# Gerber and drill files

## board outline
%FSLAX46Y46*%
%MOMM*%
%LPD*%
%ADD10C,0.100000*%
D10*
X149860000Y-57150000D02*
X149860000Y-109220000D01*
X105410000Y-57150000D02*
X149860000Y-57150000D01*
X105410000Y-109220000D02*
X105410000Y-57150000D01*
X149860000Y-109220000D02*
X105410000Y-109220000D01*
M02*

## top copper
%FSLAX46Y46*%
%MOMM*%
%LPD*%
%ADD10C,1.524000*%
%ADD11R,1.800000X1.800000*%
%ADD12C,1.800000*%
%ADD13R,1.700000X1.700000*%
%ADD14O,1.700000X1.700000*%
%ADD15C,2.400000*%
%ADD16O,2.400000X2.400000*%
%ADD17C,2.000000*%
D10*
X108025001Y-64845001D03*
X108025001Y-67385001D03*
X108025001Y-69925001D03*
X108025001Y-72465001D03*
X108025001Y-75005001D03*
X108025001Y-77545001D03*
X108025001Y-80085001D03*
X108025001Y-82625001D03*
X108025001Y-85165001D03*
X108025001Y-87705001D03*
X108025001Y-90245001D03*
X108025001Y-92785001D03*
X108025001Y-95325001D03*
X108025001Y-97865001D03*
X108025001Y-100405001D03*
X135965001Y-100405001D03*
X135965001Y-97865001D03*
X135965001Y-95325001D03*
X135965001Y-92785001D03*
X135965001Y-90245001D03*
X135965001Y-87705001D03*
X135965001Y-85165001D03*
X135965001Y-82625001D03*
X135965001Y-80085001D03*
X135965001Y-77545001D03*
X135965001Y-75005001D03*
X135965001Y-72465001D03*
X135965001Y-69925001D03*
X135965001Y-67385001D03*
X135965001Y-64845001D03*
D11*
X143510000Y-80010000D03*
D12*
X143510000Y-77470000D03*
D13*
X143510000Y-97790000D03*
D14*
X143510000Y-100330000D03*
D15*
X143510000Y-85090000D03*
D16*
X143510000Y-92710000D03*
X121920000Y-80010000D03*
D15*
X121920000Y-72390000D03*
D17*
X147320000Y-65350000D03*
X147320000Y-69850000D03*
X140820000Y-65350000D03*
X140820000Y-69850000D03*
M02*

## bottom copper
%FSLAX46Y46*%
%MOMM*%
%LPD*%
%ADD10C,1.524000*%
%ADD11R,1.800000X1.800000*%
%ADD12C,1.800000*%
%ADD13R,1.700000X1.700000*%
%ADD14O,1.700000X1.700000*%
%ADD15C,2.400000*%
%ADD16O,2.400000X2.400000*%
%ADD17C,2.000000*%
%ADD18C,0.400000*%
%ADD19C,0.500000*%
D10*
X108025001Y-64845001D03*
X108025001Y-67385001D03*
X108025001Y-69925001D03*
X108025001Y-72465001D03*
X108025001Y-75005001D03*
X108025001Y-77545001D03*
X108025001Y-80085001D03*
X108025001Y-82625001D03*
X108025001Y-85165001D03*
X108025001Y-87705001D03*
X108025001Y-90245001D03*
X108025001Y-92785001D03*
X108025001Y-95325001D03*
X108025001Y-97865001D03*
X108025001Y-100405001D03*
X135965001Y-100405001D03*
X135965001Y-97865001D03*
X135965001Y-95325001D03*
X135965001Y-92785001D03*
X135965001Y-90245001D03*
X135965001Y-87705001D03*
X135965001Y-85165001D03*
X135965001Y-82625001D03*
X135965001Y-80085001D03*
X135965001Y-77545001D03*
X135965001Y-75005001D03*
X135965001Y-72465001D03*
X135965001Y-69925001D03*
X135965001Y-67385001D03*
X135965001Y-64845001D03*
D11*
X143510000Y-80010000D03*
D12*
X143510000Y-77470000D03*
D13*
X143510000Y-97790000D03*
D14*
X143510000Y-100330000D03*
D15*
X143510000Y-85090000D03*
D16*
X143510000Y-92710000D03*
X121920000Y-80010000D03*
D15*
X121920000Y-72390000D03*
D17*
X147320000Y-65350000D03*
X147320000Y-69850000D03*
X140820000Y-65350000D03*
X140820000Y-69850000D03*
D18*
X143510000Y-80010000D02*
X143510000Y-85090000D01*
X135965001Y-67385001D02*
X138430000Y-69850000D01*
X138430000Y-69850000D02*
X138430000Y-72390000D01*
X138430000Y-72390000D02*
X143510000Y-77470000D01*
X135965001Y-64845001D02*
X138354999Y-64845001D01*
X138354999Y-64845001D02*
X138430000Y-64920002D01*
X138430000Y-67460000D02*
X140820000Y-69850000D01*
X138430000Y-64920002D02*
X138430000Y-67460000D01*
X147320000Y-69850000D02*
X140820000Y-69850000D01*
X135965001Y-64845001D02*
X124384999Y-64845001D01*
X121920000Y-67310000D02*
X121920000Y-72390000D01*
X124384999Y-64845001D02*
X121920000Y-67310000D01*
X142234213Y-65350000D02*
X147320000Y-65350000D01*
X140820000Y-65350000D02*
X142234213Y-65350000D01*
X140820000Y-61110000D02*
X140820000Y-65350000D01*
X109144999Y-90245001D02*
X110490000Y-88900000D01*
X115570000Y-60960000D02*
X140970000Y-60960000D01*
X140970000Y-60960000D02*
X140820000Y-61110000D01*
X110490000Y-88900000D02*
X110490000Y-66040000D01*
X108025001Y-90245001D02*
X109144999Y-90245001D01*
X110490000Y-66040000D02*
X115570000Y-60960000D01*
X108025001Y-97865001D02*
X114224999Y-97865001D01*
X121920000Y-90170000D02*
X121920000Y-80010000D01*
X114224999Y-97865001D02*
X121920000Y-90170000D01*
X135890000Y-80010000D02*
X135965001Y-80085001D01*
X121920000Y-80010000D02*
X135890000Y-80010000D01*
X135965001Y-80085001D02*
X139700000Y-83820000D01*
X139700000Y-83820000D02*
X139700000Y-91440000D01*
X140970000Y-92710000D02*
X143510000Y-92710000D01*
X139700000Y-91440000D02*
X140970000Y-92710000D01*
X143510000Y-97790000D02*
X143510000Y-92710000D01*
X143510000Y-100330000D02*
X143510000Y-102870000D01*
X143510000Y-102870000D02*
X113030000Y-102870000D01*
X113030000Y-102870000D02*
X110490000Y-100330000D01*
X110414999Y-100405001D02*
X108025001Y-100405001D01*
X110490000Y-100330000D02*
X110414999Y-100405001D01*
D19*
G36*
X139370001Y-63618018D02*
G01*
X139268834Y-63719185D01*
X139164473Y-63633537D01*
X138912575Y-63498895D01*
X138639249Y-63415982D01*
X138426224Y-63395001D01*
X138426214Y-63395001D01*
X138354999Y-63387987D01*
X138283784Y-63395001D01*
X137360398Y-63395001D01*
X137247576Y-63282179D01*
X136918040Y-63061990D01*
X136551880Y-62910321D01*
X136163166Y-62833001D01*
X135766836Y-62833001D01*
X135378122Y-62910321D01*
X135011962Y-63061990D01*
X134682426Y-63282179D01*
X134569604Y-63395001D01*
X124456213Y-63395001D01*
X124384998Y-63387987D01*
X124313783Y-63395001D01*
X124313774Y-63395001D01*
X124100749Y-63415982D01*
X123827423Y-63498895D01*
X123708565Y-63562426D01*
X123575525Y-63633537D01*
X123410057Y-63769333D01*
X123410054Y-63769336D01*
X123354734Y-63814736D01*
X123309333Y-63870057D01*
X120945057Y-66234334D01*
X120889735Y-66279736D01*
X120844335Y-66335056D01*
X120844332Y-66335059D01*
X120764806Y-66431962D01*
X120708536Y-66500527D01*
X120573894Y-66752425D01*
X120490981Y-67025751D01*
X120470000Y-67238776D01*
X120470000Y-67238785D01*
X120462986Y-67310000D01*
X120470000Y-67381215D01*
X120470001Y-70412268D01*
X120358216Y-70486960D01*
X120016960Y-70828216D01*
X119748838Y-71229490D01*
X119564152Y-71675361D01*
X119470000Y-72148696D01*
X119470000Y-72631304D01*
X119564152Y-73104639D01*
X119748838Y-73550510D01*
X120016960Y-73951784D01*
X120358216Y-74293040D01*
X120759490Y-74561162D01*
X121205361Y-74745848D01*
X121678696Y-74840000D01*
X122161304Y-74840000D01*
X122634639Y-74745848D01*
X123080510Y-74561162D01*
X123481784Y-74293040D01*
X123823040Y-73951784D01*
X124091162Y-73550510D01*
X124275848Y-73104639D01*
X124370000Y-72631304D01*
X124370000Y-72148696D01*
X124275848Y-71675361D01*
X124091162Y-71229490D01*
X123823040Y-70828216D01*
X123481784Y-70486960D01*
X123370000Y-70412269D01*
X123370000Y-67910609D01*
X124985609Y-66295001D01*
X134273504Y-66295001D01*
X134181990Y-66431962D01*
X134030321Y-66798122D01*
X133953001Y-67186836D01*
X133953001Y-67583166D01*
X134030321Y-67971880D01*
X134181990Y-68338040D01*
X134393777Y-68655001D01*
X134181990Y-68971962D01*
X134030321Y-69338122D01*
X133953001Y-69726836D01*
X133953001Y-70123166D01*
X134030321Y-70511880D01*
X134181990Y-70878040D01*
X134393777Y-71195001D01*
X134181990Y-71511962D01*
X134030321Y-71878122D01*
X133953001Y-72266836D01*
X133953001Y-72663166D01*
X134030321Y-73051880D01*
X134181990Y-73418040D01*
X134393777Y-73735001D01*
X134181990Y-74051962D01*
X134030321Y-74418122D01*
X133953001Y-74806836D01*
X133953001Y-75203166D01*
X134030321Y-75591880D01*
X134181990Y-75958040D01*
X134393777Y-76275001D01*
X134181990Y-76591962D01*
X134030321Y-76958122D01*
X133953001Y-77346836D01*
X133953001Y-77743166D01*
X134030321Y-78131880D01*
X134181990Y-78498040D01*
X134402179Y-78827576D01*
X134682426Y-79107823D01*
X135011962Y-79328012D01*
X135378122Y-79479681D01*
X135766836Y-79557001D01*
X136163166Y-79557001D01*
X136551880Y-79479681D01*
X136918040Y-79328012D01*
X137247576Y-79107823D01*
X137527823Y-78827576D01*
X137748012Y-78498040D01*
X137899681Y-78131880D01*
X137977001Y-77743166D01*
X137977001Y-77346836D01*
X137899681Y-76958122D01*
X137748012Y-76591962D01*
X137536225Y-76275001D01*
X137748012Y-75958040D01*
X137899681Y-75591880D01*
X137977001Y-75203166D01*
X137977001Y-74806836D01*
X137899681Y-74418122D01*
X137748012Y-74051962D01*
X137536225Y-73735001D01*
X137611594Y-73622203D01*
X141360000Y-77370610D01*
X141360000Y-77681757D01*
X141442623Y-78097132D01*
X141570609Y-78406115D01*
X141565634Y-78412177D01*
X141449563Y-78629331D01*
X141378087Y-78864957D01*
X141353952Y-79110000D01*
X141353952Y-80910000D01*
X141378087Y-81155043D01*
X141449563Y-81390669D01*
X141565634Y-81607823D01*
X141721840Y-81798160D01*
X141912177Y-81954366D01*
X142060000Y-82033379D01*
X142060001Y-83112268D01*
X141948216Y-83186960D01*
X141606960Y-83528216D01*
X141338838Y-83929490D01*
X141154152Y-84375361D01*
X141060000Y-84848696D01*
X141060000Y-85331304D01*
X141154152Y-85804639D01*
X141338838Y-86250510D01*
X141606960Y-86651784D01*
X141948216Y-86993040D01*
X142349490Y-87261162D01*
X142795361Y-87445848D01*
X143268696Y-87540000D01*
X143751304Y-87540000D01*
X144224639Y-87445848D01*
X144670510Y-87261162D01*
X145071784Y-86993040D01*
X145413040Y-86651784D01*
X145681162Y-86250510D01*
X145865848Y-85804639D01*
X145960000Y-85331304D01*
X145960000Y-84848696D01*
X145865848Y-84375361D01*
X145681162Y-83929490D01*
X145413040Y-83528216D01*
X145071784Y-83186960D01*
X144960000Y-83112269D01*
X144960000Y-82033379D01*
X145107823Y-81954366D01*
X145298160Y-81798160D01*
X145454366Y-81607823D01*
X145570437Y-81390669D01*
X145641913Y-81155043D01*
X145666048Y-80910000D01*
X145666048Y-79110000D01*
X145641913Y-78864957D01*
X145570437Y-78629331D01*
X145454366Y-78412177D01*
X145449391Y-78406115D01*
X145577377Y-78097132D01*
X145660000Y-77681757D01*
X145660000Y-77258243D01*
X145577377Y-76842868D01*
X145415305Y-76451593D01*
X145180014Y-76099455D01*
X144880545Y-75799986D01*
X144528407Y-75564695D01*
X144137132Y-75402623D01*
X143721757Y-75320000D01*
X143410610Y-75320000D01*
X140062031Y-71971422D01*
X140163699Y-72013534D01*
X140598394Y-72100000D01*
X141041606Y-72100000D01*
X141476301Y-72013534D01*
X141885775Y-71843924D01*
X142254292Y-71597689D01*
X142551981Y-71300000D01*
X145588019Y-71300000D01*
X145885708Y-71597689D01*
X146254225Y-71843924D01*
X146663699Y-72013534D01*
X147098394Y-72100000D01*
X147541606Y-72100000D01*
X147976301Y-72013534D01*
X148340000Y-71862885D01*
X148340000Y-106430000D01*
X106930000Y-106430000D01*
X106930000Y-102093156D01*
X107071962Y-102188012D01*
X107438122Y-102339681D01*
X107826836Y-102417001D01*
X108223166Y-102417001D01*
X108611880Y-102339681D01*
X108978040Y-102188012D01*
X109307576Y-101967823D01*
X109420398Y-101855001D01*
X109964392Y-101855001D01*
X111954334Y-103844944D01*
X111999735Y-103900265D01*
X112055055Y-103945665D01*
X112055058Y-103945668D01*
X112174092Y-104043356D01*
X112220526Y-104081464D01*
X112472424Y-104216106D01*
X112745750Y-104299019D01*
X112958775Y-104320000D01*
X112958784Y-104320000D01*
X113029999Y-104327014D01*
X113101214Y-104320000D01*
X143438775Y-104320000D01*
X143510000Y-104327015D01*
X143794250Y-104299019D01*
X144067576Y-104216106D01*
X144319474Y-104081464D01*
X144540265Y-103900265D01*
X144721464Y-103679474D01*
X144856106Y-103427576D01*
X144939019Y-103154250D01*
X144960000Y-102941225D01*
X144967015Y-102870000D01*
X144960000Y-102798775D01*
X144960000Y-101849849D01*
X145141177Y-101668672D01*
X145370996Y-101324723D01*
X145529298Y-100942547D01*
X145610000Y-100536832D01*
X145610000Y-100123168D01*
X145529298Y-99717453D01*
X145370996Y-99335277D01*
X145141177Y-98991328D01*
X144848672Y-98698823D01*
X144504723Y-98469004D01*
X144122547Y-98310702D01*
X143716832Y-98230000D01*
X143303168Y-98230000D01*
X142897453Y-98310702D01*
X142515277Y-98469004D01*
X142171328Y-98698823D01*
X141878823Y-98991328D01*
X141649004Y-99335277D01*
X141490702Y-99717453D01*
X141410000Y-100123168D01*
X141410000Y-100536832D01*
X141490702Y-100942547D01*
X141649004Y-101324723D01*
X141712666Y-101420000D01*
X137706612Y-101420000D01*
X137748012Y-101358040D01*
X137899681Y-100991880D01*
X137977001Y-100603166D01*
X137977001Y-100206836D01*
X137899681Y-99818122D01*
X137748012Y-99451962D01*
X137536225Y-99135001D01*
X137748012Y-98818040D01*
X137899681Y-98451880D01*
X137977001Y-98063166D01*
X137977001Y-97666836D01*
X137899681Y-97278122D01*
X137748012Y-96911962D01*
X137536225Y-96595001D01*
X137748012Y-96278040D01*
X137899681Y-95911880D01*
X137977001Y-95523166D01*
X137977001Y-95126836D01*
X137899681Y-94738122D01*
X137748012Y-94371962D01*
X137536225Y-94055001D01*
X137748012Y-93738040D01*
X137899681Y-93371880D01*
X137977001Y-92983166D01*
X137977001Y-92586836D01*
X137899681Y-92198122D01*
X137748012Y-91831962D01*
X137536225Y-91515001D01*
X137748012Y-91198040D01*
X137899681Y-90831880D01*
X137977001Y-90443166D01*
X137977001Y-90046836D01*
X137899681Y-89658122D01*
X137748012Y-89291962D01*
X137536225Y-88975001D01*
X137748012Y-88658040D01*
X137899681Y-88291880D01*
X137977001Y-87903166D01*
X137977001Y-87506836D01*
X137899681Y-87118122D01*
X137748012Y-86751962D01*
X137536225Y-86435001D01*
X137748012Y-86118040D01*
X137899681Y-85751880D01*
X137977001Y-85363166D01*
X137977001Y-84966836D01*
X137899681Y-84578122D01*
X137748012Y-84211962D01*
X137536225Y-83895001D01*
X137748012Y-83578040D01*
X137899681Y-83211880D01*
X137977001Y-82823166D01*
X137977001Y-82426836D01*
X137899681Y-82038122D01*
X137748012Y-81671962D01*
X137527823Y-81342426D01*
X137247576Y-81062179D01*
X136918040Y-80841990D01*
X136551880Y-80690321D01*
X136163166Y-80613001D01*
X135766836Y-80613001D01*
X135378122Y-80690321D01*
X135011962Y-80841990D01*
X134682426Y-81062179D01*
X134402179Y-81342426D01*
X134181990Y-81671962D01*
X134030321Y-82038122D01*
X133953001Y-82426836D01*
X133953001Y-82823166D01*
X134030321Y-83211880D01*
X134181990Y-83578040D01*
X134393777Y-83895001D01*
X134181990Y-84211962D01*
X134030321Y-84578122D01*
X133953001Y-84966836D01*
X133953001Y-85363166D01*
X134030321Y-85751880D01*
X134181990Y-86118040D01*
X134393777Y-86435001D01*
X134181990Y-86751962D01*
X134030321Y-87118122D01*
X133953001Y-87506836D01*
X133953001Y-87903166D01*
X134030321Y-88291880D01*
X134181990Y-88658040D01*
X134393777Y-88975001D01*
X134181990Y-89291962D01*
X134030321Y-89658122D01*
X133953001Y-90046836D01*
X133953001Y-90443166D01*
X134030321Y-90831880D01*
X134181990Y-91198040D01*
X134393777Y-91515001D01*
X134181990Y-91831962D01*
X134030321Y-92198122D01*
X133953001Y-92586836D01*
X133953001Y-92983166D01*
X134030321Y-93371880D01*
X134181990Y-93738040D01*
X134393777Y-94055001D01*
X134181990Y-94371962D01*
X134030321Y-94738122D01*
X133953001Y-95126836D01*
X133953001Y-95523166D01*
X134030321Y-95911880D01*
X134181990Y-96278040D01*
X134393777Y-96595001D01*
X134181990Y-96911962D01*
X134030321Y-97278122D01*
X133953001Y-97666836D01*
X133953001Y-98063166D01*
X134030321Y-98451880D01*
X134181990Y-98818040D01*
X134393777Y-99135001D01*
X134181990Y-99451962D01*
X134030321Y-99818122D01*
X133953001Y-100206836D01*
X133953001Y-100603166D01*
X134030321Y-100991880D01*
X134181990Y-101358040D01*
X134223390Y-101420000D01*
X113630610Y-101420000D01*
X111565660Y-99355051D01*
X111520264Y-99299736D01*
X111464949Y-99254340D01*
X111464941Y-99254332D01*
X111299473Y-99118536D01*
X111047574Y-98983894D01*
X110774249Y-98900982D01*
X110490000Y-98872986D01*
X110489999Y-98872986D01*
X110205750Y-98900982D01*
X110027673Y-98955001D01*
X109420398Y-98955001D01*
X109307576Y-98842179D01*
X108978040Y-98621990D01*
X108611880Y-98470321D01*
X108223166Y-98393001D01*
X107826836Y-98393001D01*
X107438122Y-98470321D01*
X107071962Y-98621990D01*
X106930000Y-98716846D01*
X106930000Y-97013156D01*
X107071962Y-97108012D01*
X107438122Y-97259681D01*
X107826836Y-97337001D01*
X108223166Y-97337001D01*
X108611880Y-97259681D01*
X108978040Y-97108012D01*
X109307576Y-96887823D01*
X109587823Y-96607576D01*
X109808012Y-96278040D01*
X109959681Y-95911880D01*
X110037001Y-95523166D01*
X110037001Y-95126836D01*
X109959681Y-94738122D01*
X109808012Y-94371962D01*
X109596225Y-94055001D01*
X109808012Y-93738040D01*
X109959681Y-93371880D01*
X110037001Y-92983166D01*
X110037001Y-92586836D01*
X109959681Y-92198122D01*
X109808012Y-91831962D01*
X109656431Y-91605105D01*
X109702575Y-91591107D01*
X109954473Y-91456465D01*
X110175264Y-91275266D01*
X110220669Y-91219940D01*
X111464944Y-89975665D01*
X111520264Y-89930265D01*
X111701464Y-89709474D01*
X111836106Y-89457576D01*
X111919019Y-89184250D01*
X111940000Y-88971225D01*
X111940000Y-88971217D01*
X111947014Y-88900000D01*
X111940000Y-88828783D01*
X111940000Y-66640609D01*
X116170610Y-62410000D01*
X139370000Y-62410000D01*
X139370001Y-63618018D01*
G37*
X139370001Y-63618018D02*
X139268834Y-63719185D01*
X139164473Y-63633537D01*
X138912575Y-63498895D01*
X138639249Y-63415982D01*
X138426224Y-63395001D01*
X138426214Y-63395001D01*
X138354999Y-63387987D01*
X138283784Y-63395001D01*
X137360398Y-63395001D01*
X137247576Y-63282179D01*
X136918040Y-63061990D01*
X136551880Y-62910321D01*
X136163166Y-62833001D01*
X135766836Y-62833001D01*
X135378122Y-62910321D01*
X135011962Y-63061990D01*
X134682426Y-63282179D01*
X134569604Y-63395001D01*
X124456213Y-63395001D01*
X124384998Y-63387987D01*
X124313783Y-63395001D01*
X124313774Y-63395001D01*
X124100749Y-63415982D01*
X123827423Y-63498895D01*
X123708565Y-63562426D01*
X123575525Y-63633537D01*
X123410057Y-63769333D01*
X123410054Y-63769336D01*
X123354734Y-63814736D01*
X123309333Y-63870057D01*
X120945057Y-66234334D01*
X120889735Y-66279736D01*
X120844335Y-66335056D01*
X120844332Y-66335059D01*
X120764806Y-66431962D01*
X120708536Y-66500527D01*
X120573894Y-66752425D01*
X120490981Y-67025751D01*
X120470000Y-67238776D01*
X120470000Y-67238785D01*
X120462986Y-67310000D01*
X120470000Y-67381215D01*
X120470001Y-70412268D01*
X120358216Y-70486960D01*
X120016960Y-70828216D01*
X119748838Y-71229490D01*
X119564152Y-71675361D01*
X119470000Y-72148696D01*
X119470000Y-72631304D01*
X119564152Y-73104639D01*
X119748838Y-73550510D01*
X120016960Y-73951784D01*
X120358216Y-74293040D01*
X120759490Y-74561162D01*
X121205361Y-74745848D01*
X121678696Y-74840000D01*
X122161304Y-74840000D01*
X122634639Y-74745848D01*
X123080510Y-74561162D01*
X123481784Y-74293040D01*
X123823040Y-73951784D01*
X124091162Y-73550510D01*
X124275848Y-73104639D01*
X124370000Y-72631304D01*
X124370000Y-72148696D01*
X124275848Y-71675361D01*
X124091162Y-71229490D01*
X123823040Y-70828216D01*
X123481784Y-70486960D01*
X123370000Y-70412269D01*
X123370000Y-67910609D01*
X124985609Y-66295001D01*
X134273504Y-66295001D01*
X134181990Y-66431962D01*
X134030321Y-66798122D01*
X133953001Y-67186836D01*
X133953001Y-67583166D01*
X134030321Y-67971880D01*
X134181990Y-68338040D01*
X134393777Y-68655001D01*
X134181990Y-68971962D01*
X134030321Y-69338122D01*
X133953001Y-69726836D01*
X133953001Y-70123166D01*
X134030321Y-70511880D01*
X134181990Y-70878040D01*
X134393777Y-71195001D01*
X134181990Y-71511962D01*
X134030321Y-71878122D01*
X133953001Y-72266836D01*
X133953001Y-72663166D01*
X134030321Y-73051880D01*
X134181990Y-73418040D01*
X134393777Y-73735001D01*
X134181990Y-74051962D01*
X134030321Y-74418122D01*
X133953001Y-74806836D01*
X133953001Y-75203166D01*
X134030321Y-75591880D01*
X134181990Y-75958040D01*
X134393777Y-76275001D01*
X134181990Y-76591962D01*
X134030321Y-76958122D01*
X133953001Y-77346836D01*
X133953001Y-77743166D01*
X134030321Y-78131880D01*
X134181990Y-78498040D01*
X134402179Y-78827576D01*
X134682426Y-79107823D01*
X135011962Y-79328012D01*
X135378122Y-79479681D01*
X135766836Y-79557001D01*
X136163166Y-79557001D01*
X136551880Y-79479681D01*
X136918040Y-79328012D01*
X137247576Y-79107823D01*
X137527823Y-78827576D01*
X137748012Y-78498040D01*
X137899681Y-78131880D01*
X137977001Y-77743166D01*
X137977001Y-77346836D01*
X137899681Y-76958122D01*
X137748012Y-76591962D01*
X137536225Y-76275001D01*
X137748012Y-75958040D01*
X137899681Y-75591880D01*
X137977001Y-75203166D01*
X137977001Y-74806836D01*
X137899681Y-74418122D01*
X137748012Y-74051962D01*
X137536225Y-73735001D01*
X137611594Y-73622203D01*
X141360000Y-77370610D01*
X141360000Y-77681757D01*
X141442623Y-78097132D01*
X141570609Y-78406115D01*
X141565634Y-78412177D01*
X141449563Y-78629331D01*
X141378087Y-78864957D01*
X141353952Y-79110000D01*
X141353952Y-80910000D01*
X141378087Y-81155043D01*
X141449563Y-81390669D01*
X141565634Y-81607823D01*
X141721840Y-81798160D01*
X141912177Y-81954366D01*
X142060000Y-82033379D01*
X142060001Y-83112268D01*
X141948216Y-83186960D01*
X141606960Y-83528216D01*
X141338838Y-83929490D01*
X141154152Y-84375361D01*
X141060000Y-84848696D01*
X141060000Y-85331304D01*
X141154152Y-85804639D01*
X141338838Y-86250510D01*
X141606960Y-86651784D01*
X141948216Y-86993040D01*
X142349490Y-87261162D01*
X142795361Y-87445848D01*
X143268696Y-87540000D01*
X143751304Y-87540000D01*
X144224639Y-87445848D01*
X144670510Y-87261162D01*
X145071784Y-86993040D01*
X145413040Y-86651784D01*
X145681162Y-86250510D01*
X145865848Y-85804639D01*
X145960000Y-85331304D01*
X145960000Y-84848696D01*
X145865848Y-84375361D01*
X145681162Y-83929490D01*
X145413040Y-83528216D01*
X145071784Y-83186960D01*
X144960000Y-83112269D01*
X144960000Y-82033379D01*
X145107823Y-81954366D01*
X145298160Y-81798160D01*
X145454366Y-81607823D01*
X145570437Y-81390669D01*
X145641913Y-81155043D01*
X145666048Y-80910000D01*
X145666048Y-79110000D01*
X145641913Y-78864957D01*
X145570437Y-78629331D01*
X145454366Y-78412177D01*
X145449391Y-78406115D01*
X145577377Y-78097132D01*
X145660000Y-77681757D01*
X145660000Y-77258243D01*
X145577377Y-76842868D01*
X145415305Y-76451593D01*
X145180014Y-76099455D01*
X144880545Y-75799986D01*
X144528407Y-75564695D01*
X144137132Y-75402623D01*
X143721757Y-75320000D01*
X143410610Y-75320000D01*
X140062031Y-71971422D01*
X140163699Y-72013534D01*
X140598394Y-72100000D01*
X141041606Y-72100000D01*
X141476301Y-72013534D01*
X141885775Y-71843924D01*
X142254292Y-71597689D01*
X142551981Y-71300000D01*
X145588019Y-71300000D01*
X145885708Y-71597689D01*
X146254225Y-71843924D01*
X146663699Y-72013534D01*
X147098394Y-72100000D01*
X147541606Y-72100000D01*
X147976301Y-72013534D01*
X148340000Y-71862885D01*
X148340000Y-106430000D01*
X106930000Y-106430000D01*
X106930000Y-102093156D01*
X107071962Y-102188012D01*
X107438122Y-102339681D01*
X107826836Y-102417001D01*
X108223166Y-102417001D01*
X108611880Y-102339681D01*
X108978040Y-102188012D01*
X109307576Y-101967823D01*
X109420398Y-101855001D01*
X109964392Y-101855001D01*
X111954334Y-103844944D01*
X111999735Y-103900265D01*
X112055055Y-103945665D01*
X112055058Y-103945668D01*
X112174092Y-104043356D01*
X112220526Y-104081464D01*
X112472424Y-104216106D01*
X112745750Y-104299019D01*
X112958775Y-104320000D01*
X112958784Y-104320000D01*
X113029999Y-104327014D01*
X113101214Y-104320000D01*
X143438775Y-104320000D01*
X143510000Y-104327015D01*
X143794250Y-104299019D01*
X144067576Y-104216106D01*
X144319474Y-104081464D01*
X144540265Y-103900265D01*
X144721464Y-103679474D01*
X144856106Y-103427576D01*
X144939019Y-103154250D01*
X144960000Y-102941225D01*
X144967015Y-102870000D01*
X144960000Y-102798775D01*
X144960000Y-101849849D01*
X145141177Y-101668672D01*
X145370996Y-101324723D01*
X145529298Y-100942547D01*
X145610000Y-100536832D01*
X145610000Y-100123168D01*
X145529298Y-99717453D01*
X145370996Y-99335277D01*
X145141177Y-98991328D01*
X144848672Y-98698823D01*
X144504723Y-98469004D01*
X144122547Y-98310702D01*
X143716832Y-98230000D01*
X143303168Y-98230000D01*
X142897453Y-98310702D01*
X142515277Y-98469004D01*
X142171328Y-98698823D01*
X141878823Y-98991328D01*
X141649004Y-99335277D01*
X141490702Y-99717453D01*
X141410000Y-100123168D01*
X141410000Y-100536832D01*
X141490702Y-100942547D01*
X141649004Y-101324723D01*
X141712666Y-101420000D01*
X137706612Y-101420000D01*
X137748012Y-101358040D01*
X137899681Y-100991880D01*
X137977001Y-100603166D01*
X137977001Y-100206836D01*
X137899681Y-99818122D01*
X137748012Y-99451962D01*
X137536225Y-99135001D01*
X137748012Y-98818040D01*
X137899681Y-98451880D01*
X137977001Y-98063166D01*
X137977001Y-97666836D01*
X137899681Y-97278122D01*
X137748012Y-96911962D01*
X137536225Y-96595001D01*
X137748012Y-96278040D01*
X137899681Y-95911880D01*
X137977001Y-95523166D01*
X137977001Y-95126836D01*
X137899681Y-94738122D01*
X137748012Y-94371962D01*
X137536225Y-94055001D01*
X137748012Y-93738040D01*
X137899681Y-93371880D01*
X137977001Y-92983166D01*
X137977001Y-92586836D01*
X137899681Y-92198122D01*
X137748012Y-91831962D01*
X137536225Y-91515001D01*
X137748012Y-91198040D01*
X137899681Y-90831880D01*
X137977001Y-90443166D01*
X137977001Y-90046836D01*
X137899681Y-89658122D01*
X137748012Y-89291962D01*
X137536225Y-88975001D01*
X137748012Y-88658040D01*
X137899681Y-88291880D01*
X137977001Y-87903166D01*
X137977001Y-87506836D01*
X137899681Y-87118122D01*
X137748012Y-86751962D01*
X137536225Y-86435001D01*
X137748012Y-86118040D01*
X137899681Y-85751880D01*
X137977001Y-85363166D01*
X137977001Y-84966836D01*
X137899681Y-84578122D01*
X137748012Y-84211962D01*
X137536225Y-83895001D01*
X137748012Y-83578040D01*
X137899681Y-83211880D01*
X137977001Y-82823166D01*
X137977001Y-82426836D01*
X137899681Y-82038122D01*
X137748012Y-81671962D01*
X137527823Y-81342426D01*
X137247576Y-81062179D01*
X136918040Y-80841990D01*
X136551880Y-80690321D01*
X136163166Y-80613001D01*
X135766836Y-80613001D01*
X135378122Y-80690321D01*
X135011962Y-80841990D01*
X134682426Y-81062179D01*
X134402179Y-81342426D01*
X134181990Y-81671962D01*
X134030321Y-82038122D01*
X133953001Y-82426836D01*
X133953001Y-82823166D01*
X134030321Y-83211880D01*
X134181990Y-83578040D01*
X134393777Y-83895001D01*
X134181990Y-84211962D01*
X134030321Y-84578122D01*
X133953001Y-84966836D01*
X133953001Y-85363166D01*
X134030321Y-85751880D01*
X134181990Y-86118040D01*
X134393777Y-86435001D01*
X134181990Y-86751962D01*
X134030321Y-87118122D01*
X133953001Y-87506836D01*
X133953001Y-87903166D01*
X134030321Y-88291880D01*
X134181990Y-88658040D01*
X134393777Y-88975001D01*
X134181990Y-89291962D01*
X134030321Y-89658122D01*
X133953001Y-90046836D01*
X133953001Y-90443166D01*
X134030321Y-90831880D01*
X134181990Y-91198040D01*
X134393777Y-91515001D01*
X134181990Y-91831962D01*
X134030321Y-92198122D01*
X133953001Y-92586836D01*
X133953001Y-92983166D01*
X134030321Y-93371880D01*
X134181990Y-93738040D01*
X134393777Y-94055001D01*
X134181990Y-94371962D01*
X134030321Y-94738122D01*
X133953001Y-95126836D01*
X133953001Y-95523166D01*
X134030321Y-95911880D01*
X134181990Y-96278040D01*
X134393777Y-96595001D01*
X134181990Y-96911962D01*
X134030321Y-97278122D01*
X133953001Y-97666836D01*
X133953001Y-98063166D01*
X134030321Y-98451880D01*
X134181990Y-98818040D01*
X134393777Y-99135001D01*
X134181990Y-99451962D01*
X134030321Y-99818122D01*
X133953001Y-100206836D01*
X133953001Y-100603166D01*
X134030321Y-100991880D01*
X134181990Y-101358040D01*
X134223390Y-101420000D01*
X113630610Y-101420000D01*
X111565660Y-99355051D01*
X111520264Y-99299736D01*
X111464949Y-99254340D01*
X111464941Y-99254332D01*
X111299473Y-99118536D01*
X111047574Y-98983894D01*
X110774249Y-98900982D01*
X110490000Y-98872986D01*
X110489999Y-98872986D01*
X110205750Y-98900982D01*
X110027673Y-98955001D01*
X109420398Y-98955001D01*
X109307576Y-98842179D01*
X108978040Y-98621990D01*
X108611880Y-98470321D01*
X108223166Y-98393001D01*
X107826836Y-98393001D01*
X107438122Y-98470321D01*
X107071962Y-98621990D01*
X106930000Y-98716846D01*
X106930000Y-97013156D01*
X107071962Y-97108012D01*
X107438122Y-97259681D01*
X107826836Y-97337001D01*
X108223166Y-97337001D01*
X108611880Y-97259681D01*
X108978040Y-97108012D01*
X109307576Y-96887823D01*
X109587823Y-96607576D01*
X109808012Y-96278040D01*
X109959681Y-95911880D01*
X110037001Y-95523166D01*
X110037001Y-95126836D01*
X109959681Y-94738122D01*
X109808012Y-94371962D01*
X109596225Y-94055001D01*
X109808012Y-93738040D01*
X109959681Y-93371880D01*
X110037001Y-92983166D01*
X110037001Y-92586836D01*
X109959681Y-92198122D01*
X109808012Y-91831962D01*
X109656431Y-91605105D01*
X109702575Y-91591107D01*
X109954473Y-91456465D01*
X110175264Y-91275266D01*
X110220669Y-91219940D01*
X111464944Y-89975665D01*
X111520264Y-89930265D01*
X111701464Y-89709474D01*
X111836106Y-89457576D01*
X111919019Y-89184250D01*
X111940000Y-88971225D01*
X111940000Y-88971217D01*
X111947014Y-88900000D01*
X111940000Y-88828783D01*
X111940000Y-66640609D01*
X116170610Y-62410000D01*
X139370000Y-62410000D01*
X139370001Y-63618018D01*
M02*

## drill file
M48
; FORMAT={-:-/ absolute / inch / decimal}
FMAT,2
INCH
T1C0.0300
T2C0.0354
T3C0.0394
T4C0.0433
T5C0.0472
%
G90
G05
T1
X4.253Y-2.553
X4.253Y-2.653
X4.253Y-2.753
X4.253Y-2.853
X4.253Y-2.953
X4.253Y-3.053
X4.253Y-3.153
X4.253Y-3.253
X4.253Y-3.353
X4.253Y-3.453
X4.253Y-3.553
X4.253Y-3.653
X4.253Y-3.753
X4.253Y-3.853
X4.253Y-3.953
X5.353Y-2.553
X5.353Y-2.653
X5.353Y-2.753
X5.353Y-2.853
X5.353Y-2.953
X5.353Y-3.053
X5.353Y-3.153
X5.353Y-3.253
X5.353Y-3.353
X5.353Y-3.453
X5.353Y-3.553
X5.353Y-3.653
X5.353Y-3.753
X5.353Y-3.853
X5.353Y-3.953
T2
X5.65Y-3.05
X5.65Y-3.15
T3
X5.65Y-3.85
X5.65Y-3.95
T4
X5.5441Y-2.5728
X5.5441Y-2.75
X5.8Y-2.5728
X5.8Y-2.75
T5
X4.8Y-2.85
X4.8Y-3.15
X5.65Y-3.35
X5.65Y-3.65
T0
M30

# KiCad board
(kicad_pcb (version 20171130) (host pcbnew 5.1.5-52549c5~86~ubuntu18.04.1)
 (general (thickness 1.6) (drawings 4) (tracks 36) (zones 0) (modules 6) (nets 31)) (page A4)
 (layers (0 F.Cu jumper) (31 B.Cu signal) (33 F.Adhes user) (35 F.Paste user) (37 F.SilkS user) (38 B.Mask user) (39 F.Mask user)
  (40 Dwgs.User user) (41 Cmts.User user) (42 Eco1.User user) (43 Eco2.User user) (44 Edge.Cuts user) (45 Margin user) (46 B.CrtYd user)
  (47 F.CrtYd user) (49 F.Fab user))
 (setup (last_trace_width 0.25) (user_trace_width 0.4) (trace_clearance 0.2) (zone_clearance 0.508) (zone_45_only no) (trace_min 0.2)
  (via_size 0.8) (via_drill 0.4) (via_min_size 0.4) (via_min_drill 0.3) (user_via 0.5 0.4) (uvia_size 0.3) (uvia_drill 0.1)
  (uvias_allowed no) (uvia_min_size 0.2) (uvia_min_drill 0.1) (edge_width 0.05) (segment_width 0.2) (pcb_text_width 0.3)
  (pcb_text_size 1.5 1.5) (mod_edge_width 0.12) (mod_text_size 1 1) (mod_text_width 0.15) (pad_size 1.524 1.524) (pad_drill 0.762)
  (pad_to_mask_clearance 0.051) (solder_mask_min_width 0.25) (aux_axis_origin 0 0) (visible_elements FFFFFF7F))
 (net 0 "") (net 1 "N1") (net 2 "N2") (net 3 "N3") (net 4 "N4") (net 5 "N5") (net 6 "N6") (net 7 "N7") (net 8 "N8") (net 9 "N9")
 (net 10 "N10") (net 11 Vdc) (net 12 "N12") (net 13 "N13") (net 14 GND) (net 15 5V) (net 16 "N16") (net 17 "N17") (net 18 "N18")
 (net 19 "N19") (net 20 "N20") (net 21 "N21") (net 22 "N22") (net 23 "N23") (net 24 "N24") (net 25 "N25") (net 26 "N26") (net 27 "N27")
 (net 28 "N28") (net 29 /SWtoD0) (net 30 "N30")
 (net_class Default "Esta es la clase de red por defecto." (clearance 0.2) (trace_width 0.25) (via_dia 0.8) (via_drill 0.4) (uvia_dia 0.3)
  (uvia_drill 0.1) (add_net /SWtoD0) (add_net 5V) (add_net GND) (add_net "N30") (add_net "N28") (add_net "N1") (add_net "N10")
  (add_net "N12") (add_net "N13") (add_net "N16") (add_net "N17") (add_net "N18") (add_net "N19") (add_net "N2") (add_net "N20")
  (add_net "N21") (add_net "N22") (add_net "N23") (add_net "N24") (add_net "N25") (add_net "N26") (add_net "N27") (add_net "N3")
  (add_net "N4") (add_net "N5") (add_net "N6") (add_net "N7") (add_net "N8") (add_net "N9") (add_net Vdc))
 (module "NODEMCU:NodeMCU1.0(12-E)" (layer F.Cu) (at 121.995001 82.625001)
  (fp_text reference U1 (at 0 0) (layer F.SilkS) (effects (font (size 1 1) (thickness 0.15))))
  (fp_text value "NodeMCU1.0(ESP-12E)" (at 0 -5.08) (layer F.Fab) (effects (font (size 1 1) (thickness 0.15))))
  (pad 1 thru_hole circle (at -13.97 -17.78) (size 1.524 1.524) (drill 0.762) (layers *.Cu *.Mask F.SilkS) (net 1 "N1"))
  (pad 2 thru_hole circle (at -13.97 -15.24) (size 1.524 1.524) (drill 0.762) (layers *.Cu *.Mask F.SilkS) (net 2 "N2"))
  (pad 3 thru_hole circle (at -13.97 -12.7) (size 1.524 1.524) (drill 0.762) (layers *.Cu *.Mask F.SilkS) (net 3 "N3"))
  (pad 4 thru_hole circle (at -13.97 -10.16) (size 1.524 1.524) (drill 0.762) (layers *.Cu *.Mask F.SilkS) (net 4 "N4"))
  (pad 5 thru_hole circle (at -13.97 -7.62) (size 1.524 1.524) (drill 0.762) (layers *.Cu *.Mask F.SilkS) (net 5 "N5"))
  (pad 6 thru_hole circle (at -13.97 -5.08) (size 1.524 1.524) (drill 0.762) (layers *.Cu *.Mask F.SilkS) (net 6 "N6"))
  (pad 7 thru_hole circle (at -13.97 -2.54) (size 1.524 1.524) (drill 0.762) (layers *.Cu *.Mask F.SilkS) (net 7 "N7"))
  (pad 8 thru_hole circle (at -13.97 0) (size 1.524 1.524) (drill 0.762) (layers *.Cu *.Mask F.SilkS) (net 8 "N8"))
  (pad 9 thru_hole circle (at -13.97 2.54) (size 1.524 1.524) (drill 0.762) (layers *.Cu *.Mask F.SilkS) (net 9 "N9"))
  (pad 10 thru_hole circle (at -13.97 5.08) (size 1.524 1.524) (drill 0.762) (layers *.Cu *.Mask F.SilkS) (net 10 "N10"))
  (pad 11 thru_hole circle (at -13.97 7.62) (size 1.524 1.524) (drill 0.762) (layers *.Cu *.Mask F.SilkS) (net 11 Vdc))
  (pad 12 thru_hole circle (at -13.97 10.16) (size 1.524 1.524) (drill 0.762) (layers *.Cu *.Mask F.SilkS) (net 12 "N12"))
  (pad 13 thru_hole circle (at -13.97 12.7) (size 1.524 1.524) (drill 0.762) (layers *.Cu *.Mask F.SilkS) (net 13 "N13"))
  (pad 14 thru_hole circle (at -13.97 15.24) (size 1.524 1.524) (drill 0.762) (layers *.Cu *.Mask F.SilkS) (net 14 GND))
  (pad 15 thru_hole circle (at -13.97 17.78) (size 1.524 1.524) (drill 0.762) (layers *.Cu *.Mask F.SilkS) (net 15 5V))
  (pad 16 thru_hole circle (at 13.97 17.78) (size 1.524 1.524) (drill 0.762) (layers *.Cu *.Mask F.SilkS) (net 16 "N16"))
  (pad 17 thru_hole circle (at 13.97 15.24) (size 1.524 1.524) (drill 0.762) (layers *.Cu *.Mask F.SilkS) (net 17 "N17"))
  (pad 18 thru_hole circle (at 13.97 12.7) (size 1.524 1.524) (drill 0.762) (layers *.Cu *.Mask F.SilkS) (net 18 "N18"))
  (pad 19 thru_hole circle (at 13.97 10.16) (size 1.524 1.524) (drill 0.762) (layers *.Cu *.Mask F.SilkS) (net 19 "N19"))
  (pad 20 thru_hole circle (at 13.97 7.62) (size 1.524 1.524) (drill 0.762) (layers *.Cu *.Mask F.SilkS) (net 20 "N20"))
  (pad 21 thru_hole circle (at 13.97 5.08) (size 1.524 1.524) (drill 0.762) (layers *.Cu *.Mask F.SilkS) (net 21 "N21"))
  (pad 22 thru_hole circle (at 13.97 2.54) (size 1.524 1.524) (drill 0.762) (layers *.Cu *.Mask F.SilkS) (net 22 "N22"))
  (pad 23 thru_hole circle (at 13.97 0) (size 1.524 1.524) (drill 0.762) (layers *.Cu *.Mask F.SilkS) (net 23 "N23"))
  (pad 24 thru_hole circle (at 13.97 -2.54) (size 1.524 1.524) (drill 0.762) (layers *.Cu *.Mask F.SilkS) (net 14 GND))
  (pad 25 thru_hole circle (at 13.97 -5.08) (size 1.524 1.524) (drill 0.762) (layers *.Cu *.Mask F.SilkS) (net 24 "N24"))
  (pad 26 thru_hole circle (at 13.97 -7.62) (size 1.524 1.524) (drill 0.762) (layers *.Cu *.Mask F.SilkS) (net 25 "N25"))
  (pad 27 thru_hole circle (at 13.97 -10.16) (size 1.524 1.524) (drill 0.762) (layers *.Cu *.Mask F.SilkS) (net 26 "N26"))
  (pad 28 thru_hole circle (at 13.97 -12.7) (size 1.524 1.524) (drill 0.762) (layers *.Cu *.Mask F.SilkS) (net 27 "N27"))
  (pad 29 thru_hole circle (at 13.97 -15.24) (size 1.524 1.524) (drill 0.762) (layers *.Cu *.Mask F.SilkS) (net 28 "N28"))
  (pad 30 thru_hole circle (at 13.97 -17.78) (size 1.524 1.524) (drill 0.762) (layers *.Cu *.Mask F.SilkS) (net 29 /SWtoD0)))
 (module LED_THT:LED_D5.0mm (layer F.Cu) (at 143.51 80.01 90)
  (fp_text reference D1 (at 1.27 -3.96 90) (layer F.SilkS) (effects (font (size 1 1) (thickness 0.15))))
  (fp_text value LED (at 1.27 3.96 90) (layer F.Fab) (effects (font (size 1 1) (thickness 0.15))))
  (pad 1 thru_hole rect (at 0 0 90) (size 1.8 1.8) (drill 0.9) (layers *.Cu *.Mask) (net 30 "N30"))
  (pad 2 thru_hole circle (at 2.54 0 90) (size 1.8 1.8) (drill 0.9) (layers *.Cu *.Mask) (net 28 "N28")))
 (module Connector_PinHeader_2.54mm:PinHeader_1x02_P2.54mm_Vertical (layer F.Cu) (at 143.51 97.79)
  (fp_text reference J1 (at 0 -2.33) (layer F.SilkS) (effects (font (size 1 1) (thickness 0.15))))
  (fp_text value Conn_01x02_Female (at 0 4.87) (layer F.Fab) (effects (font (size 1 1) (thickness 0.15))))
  (pad 1 thru_hole rect (at 0 0) (size 1.7 1.7) (drill 1) (layers *.Cu *.Mask) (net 14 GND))
  (pad 2 thru_hole oval (at 0 2.54) (size 1.7 1.7) (drill 1) (layers *.Cu *.Mask) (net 15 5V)))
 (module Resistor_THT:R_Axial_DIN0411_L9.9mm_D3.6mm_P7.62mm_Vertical (layer F.Cu) (at 143.51 85.09 270)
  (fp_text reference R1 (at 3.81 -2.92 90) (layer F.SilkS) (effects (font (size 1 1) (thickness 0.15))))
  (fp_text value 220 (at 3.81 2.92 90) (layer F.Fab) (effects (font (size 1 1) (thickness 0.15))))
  (pad 1 thru_hole circle (at 0 0 270) (size 2.4 2.4) (drill 1.2) (layers *.Cu *.Mask) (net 30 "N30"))
  (pad 2 thru_hole oval (at 7.62 0 270) (size 2.4 2.4) (drill 1.2) (layers *.Cu *.Mask) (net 14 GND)))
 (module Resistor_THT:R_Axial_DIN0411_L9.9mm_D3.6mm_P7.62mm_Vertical (layer F.Cu) (at 121.92 72.39 270)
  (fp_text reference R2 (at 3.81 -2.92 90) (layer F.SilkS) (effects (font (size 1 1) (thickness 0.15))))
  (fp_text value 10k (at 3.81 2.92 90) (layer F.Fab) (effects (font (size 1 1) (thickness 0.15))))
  (pad 2 thru_hole oval (at 7.62 0 270) (size 2.4 2.4) (drill 1.2) (layers *.Cu *.Mask) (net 14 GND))
  (pad 1 thru_hole circle (at 0 0 270) (size 2.4 2.4) (drill 1.2) (layers *.Cu *.Mask) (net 29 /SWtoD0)))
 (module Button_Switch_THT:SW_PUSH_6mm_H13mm (layer F.Cu) (at 147.32 69.85 180)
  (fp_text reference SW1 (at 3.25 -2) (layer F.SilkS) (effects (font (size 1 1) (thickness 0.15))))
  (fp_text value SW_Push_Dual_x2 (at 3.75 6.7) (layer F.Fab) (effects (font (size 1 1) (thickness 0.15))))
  (pad 2 thru_hole circle (at 0 4.5 270) (size 2 2) (drill 1.1) (layers *.Cu *.Mask) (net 11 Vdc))
  (pad 1 thru_hole circle (at 0 0 270) (size 2 2) (drill 1.1) (layers *.Cu *.Mask) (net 29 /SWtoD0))
  (pad 2 thru_hole circle (at 6.5 4.5 270) (size 2 2) (drill 1.1) (layers *.Cu *.Mask) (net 11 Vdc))
  (pad 1 thru_hole circle (at 6.5 0 270) (size 2 2) (drill 1.1) (layers *.Cu *.Mask) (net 29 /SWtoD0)))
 (gr_line (start 149.86 57.15) (end 149.86 109.22) (layer Edge.Cuts) (width 0.1))
 (gr_line (start 105.41 57.15) (end 149.86 57.15) (layer Edge.Cuts) (width 0.1))
 (gr_line (start 105.41 109.22) (end 105.41 57.15) (layer Edge.Cuts) (width 0.1))
 (gr_line (start 149.86 109.22) (end 105.41 109.22) (layer Edge.Cuts) (width 0.1))
 (segment (start 143.51 80.01) (end 143.51 85.09) (width 0.4) (layer B.Cu) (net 30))
 (segment (start 135.965001 67.385001) (end 138.43 69.85) (width 0.4) (layer B.Cu) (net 28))
 (segment (start 138.43 69.85) (end 138.43 72.39) (width 0.4) (layer B.Cu) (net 28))
 (segment (start 138.43 72.39) (end 143.51 77.47) (width 0.4) (layer B.Cu) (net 28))
 (segment (start 135.965001 64.845001) (end 138.354999 64.845001) (width 0.4) (layer B.Cu) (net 29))
 (segment (start 138.354999 64.845001) (end 138.43 64.920002) (width 0.4) (layer B.Cu) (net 29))
 (segment (start 138.43 67.46) (end 140.82 69.85) (width 0.4) (layer B.Cu) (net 29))
 (segment (start 138.43 64.920002) (end 138.43 67.46) (width 0.4) (layer B.Cu) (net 29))
 (segment (start 147.32 69.85) (end 140.82 69.85) (width 0.4) (layer B.Cu) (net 29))
 (segment (start 135.965001 64.845001) (end 124.384999 64.845001) (width 0.4) (layer B.Cu) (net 29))
 (segment (start 121.92 67.31) (end 121.92 72.39) (width 0.4) (layer B.Cu) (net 29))
 (segment (start 124.384999 64.845001) (end 121.92 67.31) (width 0.4) (layer B.Cu) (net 29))
 (segment (start 142.234213 65.35) (end 147.32 65.35) (width 0.4) (layer B.Cu) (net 11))
 (segment (start 140.82 65.35) (end 142.234213 65.35) (width 0.4) (layer B.Cu) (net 11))
 (segment (start 140.82 61.11) (end 140.82 65.35) (width 0.4) (layer B.Cu) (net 11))
 (segment (start 109.144999 90.245001) (end 110.49 88.9) (width 0.4) (layer B.Cu) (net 11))
 (segment (start 115.57 60.96) (end 140.97 60.96) (width 0.4) (layer B.Cu) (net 11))
 (segment (start 140.97 60.96) (end 140.82 61.11) (width 0.4) (layer B.Cu) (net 11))
 (segment (start 110.49 88.9) (end 110.49 66.04) (width 0.4) (layer B.Cu) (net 11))
 (segment (start 108.025001 90.245001) (end 109.144999 90.245001) (width 0.4) (layer B.Cu) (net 11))
 (segment (start 110.49 66.04) (end 115.57 60.96) (width 0.4) (layer B.Cu) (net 11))
 (segment (start 108.025001 97.865001) (end 114.224999 97.865001) (width 0.4) (layer B.Cu) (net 14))
 (segment (start 121.92 90.17) (end 121.92 80.01) (width 0.4) (layer B.Cu) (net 14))
 (segment (start 114.224999 97.865001) (end 121.92 90.17) (width 0.4) (layer B.Cu) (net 14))
 (segment (start 135.89 80.01) (end 135.965001 80.085001) (width 0.4) (layer B.Cu) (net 14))
 (segment (start 121.92 80.01) (end 135.89 80.01) (width 0.4) (layer B.Cu) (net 14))
 (segment (start 135.965001 80.085001) (end 139.7 83.82) (width 0.4) (layer B.Cu) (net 14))
 (segment (start 139.7 83.82) (end 139.7 91.44) (width 0.4) (layer B.Cu) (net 14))
 (segment (start 140.97 92.71) (end 143.51 92.71) (width 0.4) (layer B.Cu) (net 14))
 (segment (start 139.7 91.44) (end 140.97 92.71) (width 0.4) (layer B.Cu) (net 14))
 (segment (start 143.51 97.79) (end 143.51 92.71) (width 0.4) (layer B.Cu) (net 14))
 (segment (start 143.51 100.33) (end 143.51 102.87) (width 0.4) (layer B.Cu) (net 15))
 (segment (start 143.51 102.87) (end 113.03 102.87) (width 0.4) (layer B.Cu) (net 15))
 (segment (start 113.03 102.87) (end 110.49 100.33) (width 0.4) (layer B.Cu) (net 15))
 (segment (start 110.414999 100.405001) (end 108.025001 100.405001) (width 0.4) (layer B.Cu) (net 15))
 (segment (start 110.49 100.33) (end 110.414999 100.405001) (width 0.4) (layer B.Cu) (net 15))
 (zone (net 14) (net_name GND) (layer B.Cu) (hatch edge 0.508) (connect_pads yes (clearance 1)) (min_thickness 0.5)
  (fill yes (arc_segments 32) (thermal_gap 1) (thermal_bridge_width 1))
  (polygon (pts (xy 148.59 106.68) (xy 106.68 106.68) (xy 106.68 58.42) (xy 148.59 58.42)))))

